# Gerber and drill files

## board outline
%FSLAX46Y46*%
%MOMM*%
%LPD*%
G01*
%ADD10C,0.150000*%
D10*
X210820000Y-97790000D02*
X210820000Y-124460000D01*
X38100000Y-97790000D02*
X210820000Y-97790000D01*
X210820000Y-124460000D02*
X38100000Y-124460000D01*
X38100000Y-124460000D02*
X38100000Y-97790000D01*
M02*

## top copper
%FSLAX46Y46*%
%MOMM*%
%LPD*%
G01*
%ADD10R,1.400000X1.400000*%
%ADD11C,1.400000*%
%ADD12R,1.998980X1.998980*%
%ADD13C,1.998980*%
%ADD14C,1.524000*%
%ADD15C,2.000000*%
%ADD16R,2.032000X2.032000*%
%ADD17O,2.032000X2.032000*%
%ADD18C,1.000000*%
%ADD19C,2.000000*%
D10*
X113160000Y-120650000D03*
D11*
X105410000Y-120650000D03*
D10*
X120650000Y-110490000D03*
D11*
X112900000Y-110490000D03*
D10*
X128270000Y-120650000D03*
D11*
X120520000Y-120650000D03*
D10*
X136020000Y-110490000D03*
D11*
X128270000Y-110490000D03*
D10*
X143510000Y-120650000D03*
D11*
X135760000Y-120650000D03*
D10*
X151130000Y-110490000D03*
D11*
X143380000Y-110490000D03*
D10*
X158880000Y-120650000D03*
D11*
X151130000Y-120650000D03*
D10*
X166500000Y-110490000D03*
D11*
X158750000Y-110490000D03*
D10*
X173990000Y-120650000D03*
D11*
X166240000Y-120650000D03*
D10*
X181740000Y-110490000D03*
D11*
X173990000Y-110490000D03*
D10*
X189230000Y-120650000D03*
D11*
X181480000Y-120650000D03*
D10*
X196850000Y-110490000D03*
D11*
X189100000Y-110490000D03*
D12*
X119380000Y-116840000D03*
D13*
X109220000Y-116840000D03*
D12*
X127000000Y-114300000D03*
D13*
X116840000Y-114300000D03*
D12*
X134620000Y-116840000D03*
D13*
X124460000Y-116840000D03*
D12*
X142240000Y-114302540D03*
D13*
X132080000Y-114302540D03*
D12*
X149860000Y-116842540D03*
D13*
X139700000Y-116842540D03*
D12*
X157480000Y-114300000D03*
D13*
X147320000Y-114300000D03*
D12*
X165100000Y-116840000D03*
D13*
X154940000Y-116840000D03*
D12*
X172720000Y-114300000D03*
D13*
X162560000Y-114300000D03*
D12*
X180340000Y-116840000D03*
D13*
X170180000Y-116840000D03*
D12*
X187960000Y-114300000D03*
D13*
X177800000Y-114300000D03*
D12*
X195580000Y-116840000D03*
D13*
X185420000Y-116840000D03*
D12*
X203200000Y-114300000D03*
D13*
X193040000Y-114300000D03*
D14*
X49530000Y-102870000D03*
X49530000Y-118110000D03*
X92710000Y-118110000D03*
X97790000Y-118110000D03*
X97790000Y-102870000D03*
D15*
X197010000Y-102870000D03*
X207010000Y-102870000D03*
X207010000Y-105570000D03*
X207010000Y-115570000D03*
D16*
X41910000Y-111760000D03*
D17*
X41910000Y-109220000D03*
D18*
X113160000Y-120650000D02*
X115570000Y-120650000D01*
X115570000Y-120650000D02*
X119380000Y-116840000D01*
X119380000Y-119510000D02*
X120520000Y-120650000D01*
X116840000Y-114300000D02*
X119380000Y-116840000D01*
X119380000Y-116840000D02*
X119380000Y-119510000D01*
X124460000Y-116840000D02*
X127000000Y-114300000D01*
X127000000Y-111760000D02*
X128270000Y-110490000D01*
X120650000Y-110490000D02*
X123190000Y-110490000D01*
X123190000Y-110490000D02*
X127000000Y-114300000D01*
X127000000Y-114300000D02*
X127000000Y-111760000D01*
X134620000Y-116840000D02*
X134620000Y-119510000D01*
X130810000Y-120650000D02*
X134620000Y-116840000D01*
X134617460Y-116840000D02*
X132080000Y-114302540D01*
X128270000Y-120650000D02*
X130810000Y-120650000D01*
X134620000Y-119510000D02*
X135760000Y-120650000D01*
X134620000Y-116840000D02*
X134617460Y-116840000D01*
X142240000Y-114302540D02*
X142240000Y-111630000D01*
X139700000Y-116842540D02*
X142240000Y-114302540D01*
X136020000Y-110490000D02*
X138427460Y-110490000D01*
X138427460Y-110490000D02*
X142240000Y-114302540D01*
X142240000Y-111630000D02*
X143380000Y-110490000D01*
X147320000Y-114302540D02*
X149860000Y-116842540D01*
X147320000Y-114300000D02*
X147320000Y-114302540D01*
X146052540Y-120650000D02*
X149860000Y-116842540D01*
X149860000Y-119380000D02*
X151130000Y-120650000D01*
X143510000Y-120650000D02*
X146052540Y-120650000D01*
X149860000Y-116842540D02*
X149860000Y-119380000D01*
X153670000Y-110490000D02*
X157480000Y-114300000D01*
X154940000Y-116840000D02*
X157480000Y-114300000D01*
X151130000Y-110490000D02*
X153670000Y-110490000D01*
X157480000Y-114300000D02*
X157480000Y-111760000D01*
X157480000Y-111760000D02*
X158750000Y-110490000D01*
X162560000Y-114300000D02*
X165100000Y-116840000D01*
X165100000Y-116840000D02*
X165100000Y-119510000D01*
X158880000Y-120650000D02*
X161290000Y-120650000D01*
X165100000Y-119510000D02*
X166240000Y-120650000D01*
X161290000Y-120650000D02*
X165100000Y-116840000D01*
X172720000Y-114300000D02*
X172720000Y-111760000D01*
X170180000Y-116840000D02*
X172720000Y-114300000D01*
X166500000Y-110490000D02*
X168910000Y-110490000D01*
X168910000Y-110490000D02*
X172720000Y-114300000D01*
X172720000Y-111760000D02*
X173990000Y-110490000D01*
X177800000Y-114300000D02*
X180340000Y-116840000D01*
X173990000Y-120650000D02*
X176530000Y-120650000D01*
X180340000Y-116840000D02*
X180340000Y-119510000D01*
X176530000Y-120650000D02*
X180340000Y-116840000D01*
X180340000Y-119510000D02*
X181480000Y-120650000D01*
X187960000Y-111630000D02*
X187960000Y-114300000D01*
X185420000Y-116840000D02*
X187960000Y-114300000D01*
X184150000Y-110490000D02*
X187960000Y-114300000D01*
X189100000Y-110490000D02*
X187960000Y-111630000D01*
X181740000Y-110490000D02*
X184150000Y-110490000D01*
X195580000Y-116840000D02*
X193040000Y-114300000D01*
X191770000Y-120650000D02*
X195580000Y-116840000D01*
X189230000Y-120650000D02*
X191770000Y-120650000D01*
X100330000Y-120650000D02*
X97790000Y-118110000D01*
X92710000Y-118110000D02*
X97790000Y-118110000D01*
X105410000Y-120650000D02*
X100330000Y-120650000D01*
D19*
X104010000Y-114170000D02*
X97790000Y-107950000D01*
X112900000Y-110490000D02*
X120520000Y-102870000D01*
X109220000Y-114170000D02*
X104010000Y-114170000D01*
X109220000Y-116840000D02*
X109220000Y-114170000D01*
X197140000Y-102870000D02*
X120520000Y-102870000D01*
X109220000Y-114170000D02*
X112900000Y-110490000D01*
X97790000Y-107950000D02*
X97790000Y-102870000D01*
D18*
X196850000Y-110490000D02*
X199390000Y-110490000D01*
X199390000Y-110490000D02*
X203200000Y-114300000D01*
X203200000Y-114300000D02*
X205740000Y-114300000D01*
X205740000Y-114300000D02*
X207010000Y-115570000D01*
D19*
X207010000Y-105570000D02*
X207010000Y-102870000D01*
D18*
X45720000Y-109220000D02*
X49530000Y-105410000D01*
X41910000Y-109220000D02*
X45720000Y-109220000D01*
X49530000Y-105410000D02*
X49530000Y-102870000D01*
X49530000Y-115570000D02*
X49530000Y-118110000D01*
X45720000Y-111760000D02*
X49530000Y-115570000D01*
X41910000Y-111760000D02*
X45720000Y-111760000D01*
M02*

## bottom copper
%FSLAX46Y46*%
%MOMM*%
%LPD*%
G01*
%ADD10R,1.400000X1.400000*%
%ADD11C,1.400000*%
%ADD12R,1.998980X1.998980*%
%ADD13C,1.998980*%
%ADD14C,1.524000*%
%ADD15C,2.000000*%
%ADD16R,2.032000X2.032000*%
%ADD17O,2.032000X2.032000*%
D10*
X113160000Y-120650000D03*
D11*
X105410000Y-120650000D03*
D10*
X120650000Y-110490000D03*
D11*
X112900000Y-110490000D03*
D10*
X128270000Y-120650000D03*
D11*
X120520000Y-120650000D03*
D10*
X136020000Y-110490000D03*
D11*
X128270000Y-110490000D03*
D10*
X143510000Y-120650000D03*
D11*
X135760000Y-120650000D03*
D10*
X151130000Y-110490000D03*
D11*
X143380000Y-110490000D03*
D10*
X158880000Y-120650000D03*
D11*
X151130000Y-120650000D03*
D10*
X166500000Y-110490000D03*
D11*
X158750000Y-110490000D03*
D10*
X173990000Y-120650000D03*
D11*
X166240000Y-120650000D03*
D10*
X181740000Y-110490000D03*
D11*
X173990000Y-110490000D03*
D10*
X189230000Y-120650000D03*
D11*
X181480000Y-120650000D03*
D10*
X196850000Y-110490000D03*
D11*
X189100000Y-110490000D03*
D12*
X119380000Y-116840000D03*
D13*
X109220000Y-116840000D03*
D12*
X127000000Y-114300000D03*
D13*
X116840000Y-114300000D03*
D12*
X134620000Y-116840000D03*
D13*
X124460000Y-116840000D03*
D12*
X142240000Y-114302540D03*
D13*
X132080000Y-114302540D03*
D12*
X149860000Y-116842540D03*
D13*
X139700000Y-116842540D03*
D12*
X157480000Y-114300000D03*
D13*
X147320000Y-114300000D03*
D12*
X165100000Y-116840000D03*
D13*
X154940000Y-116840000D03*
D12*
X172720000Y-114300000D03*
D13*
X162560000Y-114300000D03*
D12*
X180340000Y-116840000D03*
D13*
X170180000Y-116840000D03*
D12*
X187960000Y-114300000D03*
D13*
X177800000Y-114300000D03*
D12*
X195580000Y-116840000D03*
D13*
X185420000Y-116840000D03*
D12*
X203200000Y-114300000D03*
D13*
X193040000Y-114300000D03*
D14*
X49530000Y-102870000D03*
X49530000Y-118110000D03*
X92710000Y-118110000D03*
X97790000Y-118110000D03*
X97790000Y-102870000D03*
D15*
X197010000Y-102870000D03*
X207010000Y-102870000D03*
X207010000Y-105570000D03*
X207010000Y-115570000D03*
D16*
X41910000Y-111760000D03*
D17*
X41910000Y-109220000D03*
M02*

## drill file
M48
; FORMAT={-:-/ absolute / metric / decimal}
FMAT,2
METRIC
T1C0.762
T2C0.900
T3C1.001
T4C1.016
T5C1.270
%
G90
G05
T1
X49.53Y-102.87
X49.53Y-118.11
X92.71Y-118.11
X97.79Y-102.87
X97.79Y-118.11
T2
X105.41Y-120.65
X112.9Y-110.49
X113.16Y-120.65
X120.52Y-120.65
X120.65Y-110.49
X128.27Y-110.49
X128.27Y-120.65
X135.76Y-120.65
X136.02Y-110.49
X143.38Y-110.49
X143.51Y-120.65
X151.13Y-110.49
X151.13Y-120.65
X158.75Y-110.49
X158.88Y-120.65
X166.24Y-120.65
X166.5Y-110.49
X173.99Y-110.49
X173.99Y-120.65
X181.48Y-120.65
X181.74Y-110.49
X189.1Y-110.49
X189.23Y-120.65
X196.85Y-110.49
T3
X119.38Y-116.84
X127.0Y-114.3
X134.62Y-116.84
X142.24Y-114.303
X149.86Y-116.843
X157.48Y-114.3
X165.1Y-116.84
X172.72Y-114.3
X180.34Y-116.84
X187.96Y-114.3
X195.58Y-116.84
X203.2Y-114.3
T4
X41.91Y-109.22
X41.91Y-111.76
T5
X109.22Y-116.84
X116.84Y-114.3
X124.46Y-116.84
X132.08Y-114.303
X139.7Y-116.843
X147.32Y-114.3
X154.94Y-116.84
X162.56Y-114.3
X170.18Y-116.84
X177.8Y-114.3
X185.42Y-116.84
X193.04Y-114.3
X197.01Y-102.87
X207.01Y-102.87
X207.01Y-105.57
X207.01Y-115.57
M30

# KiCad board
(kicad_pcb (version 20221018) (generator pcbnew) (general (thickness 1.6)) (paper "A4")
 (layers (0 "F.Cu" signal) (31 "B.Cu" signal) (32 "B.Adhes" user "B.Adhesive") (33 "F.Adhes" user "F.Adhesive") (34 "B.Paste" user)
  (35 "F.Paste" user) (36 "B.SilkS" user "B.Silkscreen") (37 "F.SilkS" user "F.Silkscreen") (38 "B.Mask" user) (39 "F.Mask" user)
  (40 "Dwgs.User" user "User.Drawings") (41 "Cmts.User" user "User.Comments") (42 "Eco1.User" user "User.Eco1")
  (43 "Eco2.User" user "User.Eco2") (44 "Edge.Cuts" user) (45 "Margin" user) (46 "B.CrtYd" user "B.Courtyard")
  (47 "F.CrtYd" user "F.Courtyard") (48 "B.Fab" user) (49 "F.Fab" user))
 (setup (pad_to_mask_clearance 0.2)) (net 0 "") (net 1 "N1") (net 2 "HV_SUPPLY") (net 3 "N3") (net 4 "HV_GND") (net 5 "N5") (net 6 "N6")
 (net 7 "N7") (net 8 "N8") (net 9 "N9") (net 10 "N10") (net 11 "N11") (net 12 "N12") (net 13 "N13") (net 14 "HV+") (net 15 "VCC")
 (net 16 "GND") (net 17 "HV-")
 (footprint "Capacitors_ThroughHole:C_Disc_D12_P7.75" (layer "F.Cu") (at 113.16 120.65 180)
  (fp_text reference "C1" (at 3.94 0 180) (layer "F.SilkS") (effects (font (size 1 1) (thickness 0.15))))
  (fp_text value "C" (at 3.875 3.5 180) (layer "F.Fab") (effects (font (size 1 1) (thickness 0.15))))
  (pad "1" thru_hole rect (at 0 0 180) (size 1.4 1.4) (drill 0.9) (layers "*.Cu" "*.Mask" "F.SilkS") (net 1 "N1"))
  (pad "2" thru_hole circle (at 7.75 0 180) (size 1.4 1.4) (drill 0.9) (layers "*.Cu" "*.Mask" "F.SilkS") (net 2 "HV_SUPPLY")))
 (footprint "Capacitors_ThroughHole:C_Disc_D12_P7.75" (layer "F.Cu") (at 120.65 110.49 180)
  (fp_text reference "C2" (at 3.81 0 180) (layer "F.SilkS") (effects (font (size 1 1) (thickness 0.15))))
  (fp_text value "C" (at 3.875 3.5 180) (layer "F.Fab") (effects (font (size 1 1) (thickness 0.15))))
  (pad "1" thru_hole rect (at 0 0 180) (size 1.4 1.4) (drill 0.9) (layers "*.Cu" "*.Mask" "F.SilkS") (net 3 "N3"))
  (pad "2" thru_hole circle (at 7.75 0 180) (size 1.4 1.4) (drill 0.9) (layers "*.Cu" "*.Mask" "F.SilkS") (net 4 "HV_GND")))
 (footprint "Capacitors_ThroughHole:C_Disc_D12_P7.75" (layer "F.Cu") (at 128.27 120.65 180)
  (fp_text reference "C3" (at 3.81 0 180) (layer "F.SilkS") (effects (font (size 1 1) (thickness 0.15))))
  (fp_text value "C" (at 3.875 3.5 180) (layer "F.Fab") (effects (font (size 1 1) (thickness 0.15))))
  (pad "1" thru_hole rect (at 0 0 180) (size 1.4 1.4) (drill 0.9) (layers "*.Cu" "*.Mask" "F.SilkS") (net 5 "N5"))
  (pad "2" thru_hole circle (at 7.75 0 180) (size 1.4 1.4) (drill 0.9) (layers "*.Cu" "*.Mask" "F.SilkS") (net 1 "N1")))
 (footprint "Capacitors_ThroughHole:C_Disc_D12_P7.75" (layer "F.Cu") (at 136.02 110.49 180)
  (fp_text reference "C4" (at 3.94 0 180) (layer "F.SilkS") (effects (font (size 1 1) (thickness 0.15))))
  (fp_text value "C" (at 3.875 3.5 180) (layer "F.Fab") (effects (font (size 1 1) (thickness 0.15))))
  (pad "1" thru_hole rect (at 0 0 180) (size 1.4 1.4) (drill 0.9) (layers "*.Cu" "*.Mask" "F.SilkS") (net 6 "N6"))
  (pad "2" thru_hole circle (at 7.75 0 180) (size 1.4 1.4) (drill 0.9) (layers "*.Cu" "*.Mask" "F.SilkS") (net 3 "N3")))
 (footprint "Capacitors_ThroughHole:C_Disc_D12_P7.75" (layer "F.Cu") (at 143.51 120.65 180)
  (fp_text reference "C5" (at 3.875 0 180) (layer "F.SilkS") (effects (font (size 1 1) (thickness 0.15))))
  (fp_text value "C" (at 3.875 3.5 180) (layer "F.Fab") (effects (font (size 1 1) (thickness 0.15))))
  (pad "1" thru_hole rect (at 0 0 180) (size 1.4 1.4) (drill 0.9) (layers "*.Cu" "*.Mask" "F.SilkS") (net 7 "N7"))
  (pad "2" thru_hole circle (at 7.75 0 180) (size 1.4 1.4) (drill 0.9) (layers "*.Cu" "*.Mask" "F.SilkS") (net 5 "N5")))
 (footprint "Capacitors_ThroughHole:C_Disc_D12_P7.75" (layer "F.Cu") (at 151.13 110.49 180)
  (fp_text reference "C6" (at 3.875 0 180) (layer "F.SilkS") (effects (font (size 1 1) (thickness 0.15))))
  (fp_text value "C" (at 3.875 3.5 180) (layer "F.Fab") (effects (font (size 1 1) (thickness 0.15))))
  (pad "1" thru_hole rect (at 0 0 180) (size 1.4 1.4) (drill 0.9) (layers "*.Cu" "*.Mask" "F.SilkS") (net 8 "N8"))
  (pad "2" thru_hole circle (at 7.75 0 180) (size 1.4 1.4) (drill 0.9) (layers "*.Cu" "*.Mask" "F.SilkS") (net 6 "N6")))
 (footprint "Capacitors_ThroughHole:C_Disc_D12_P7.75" (layer "F.Cu") (at 158.88 120.65 180)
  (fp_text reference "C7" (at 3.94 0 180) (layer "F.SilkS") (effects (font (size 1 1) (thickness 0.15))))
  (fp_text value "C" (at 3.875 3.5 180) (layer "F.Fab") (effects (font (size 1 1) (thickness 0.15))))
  (pad "1" thru_hole rect (at 0 0 180) (size 1.4 1.4) (drill 0.9) (layers "*.Cu" "*.Mask" "F.SilkS") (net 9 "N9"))
  (pad "2" thru_hole circle (at 7.75 0 180) (size 1.4 1.4) (drill 0.9) (layers "*.Cu" "*.Mask" "F.SilkS") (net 7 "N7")))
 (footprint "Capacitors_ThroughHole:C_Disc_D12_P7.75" (layer "F.Cu") (at 166.5 110.49 180)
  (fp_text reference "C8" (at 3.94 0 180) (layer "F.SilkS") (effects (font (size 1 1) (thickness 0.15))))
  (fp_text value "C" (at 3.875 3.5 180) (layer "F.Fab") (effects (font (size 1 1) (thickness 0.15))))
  (pad "1" thru_hole rect (at 0 0 180) (size 1.4 1.4) (drill 0.9) (layers "*.Cu" "*.Mask" "F.SilkS") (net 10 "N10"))
  (pad "2" thru_hole circle (at 7.75 0 180) (size 1.4 1.4) (drill 0.9) (layers "*.Cu" "*.Mask" "F.SilkS") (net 8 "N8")))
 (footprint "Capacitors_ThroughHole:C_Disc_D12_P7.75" (layer "F.Cu") (at 173.99 120.65 180)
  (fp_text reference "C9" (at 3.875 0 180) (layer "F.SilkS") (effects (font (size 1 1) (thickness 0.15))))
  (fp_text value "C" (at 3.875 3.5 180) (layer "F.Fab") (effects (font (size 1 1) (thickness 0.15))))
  (pad "1" thru_hole rect (at 0 0 180) (size 1.4 1.4) (drill 0.9) (layers "*.Cu" "*.Mask" "F.SilkS") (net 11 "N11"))
  (pad "2" thru_hole circle (at 7.75 0 180) (size 1.4 1.4) (drill 0.9) (layers "*.Cu" "*.Mask" "F.SilkS") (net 9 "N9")))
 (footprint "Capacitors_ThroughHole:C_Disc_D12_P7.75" (layer "F.Cu") (at 181.74 110.49 180)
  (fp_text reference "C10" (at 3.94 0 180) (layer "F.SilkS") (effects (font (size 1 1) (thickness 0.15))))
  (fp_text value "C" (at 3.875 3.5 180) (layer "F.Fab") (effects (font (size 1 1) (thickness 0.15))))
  (pad "1" thru_hole rect (at 0 0 180) (size 1.4 1.4) (drill 0.9) (layers "*.Cu" "*.Mask" "F.SilkS") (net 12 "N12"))
  (pad "2" thru_hole circle (at 7.75 0 180) (size 1.4 1.4) (drill 0.9) (layers "*.Cu" "*.Mask" "F.SilkS") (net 10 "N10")))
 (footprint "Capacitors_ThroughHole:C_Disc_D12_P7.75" (layer "F.Cu") (at 189.23 120.65 180)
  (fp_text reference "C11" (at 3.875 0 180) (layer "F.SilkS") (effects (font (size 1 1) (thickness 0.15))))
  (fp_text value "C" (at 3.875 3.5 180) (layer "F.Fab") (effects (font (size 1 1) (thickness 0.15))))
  (pad "1" thru_hole rect (at 0 0 180) (size 1.4 1.4) (drill 0.9) (layers "*.Cu" "*.Mask" "F.SilkS") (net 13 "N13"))
  (pad "2" thru_hole circle (at 7.75 0 180) (size 1.4 1.4) (drill 0.9) (layers "*.Cu" "*.Mask" "F.SilkS") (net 11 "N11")))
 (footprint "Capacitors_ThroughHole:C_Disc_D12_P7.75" (layer "F.Cu") (at 196.85 110.49 180)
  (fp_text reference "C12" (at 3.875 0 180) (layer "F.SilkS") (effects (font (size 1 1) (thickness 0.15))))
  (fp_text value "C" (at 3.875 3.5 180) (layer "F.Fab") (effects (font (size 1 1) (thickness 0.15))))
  (pad "1" thru_hole rect (at 0 0 180) (size 1.4 1.4) (drill 0.9) (layers "*.Cu" "*.Mask" "F.SilkS") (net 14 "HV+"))
  (pad "2" thru_hole circle (at 7.75 0 180) (size 1.4 1.4) (drill 0.9) (layers "*.Cu" "*.Mask" "F.SilkS") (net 12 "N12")))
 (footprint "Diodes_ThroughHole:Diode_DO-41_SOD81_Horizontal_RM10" (layer "F.Cu") (at 119.38 116.83746 180)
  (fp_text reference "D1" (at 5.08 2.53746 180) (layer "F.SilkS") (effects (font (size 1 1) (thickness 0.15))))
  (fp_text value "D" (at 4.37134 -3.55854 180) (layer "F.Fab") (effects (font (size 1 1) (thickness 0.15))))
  (pad "1" thru_hole rect (at 0 -0.00254) (size 1.99898 1.99898) (drill 1.00076) (layers "*.Cu" "*.Mask" "F.SilkS") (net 1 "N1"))
  (pad "2" thru_hole circle (at 10.16 -0.00254) (size 1.99898 1.99898) (drill 1.27) (layers "*.Cu" "*.Mask" "F.SilkS") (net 4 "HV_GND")))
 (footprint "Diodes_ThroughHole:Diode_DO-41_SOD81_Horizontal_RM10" (layer "F.Cu") (at 127 114.29746 180)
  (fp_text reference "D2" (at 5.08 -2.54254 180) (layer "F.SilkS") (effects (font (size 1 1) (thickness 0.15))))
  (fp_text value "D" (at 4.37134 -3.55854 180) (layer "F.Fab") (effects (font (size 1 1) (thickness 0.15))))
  (pad "1" thru_hole rect (at 0 -0.00254) (size 1.99898 1.99898) (drill 1.00076) (layers "*.Cu" "*.Mask" "F.SilkS") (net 3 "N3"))
  (pad "2" thru_hole circle (at 10.16 -0.00254) (size 1.99898 1.99898) (drill 1.27) (layers "*.Cu" "*.Mask" "F.SilkS") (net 1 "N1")))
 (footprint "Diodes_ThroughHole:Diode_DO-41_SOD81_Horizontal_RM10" (layer "F.Cu") (at 134.62 116.83746 180)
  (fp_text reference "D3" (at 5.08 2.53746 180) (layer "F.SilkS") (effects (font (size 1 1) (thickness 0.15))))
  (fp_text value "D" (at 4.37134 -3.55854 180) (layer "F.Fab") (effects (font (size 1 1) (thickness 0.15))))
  (pad "1" thru_hole rect (at 0 -0.00254) (size 1.99898 1.99898) (drill 1.00076) (layers "*.Cu" "*.Mask" "F.SilkS") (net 5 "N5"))
  (pad "2" thru_hole circle (at 10.16 -0.00254) (size 1.99898 1.99898) (drill 1.27) (layers "*.Cu" "*.Mask" "F.SilkS") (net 3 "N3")))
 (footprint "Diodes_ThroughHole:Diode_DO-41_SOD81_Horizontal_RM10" (layer "F.Cu") (at 142.24 114.3 180)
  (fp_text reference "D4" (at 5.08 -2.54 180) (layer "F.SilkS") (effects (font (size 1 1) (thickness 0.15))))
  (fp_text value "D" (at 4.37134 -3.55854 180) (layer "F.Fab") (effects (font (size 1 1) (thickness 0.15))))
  (pad "1" thru_hole rect (at 0 -0.00254) (size 1.99898 1.99898) (drill 1.00076) (layers "*.Cu" "*.Mask" "F.SilkS") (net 6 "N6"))
  (pad "2" thru_hole circle (at 10.16 -0.00254) (size 1.99898 1.99898) (drill 1.27) (layers "*.Cu" "*.Mask" "F.SilkS") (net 5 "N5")))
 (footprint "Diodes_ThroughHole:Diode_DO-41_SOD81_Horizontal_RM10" (layer "F.Cu") (at 149.86 116.84 180)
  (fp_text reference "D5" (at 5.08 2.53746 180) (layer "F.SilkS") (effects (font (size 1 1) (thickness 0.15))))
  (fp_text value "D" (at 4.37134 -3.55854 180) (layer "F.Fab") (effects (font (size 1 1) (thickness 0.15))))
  (pad "1" thru_hole rect (at 0 -0.00254) (size 1.99898 1.99898) (drill 1.00076) (layers "*.Cu" "*.Mask" "F.SilkS") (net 7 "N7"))
  (pad "2" thru_hole circle (at 10.16 -0.00254) (size 1.99898 1.99898) (drill 1.27) (layers "*.Cu" "*.Mask" "F.SilkS") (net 6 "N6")))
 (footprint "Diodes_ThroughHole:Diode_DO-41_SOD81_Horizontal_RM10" (layer "F.Cu") (at 157.48 114.29746 180)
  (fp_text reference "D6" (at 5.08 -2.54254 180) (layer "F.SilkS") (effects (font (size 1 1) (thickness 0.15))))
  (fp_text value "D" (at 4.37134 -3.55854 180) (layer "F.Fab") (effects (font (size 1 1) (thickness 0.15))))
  (pad "1" thru_hole rect (at 0 -0.00254) (size 1.99898 1.99898) (drill 1.00076) (layers "*.Cu" "*.Mask" "F.SilkS") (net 8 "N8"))
  (pad "2" thru_hole circle (at 10.16 -0.00254) (size 1.99898 1.99898) (drill 1.27) (layers "*.Cu" "*.Mask" "F.SilkS") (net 7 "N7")))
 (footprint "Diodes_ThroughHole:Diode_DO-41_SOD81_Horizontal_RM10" (layer "F.Cu") (at 165.1 116.83746 180)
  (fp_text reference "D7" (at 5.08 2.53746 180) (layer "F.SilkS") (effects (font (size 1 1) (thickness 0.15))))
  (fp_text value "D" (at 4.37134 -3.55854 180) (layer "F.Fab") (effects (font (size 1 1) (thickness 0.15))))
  (pad "1" thru_hole rect (at 0 -0.00254) (size 1.99898 1.99898) (drill 1.00076) (layers "*.Cu" "*.Mask" "F.SilkS") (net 9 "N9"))
  (pad "2" thru_hole circle (at 10.16 -0.00254) (size 1.99898 1.99898) (drill 1.27) (layers "*.Cu" "*.Mask" "F.SilkS") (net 8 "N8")))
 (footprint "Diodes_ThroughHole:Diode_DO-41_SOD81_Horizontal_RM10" (layer "F.Cu") (at 172.72 114.29746 180)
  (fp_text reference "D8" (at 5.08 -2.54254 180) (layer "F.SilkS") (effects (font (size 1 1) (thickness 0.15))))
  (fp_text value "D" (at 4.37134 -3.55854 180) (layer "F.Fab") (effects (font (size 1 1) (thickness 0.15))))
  (pad "1" thru_hole rect (at 0 -0.00254) (size 1.99898 1.99898) (drill 1.00076) (layers "*.Cu" "*.Mask" "F.SilkS") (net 10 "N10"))
  (pad "2" thru_hole circle (at 10.16 -0.00254) (size 1.99898 1.99898) (drill 1.27) (layers "*.Cu" "*.Mask" "F.SilkS") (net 9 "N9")))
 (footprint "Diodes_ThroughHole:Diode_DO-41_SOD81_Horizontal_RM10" (layer "F.Cu") (at 180.34 116.83746 180)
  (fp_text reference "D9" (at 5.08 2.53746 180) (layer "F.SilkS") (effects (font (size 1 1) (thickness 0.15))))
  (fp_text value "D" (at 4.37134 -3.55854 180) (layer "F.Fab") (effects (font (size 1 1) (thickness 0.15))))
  (pad "1" thru_hole rect (at 0 -0.00254) (size 1.99898 1.99898) (drill 1.00076) (layers "*.Cu" "*.Mask" "F.SilkS") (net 11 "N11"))
  (pad "2" thru_hole circle (at 10.16 -0.00254) (size 1.99898 1.99898) (drill 1.27) (layers "*.Cu" "*.Mask" "F.SilkS") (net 10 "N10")))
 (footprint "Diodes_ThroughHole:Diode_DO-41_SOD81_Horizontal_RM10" (layer "F.Cu") (at 187.96 114.29746 180)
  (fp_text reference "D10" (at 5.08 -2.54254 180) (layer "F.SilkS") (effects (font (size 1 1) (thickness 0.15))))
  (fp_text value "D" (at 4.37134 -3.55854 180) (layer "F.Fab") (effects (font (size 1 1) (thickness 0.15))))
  (pad "1" thru_hole rect (at 0 -0.00254) (size 1.99898 1.99898) (drill 1.00076) (layers "*.Cu" "*.Mask" "F.SilkS") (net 12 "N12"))
  (pad "2" thru_hole circle (at 10.16 -0.00254) (size 1.99898 1.99898) (drill 1.27) (layers "*.Cu" "*.Mask" "F.SilkS") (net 11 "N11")))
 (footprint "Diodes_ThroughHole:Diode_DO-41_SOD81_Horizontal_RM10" (layer "F.Cu") (at 195.58 116.83746 180)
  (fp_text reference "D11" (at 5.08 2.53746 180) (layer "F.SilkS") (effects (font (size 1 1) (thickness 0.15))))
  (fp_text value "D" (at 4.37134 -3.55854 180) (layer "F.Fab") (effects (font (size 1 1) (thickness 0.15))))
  (pad "1" thru_hole rect (at 0 -0.00254) (size 1.99898 1.99898) (drill 1.00076) (layers "*.Cu" "*.Mask" "F.SilkS") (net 13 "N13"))
  (pad "2" thru_hole circle (at 10.16 -0.00254) (size 1.99898 1.99898) (drill 1.27) (layers "*.Cu" "*.Mask" "F.SilkS") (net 12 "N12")))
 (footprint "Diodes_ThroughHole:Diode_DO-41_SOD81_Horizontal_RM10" (layer "F.Cu") (at 203.2 114.29746 180)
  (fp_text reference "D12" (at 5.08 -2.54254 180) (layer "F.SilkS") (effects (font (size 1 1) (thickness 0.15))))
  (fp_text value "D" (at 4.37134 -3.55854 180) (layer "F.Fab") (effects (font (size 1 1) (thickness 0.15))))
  (pad "1" thru_hole rect (at 0 -0.00254) (size 1.99898 1.99898) (drill 1.00076) (layers "*.Cu" "*.Mask" "F.SilkS") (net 14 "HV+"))
  (pad "2" thru_hole circle (at 10.16 -0.00254) (size 1.99898 1.99898) (drill 1.27) (layers "*.Cu" "*.Mask" "F.SilkS") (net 13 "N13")))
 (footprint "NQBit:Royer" (layer "F.Cu") (at 74.93 110.49)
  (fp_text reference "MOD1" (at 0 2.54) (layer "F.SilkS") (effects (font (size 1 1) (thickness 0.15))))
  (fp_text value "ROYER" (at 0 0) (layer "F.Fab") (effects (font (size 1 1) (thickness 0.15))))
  (pad "1" thru_hole circle (at -25.4 -7.62) (size 1.524 1.524) (drill 0.762) (layers "*.Cu" "*.Mask" "F.SilkS") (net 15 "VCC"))
  (pad "2" thru_hole circle (at -25.4 7.62) (size 1.524 1.524) (drill 0.762) (layers "*.Cu" "*.Mask" "F.SilkS") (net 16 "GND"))
  (pad "3" thru_hole circle (at 17.78 7.62) (size 1.524 1.524) (drill 0.762) (layers "*.Cu" "*.Mask" "F.SilkS") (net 2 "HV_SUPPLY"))
  (pad "4" thru_hole circle (at 22.86 7.62) (size 1.524 1.524) (drill 0.762) (layers "*.Cu" "*.Mask" "F.SilkS") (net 2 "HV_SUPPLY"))
  (pad "5" thru_hole circle (at 22.86 -7.62) (size 1.524 1.524) (drill 0.762) (layers "*.Cu" "*.Mask" "F.SilkS") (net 4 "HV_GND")))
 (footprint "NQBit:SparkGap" (layer "F.Cu") (at 197.01 102.87)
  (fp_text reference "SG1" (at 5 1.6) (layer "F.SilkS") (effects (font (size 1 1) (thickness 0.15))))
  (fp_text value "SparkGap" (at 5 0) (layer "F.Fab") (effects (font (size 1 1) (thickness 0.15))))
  (pad "1" thru_hole circle (at 0 0) (size 2 2) (drill 1.27) (layers "*.Cu" "*.Mask" "F.SilkS") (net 4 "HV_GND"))
  (pad "2" thru_hole circle (at 10 0) (size 2 2) (drill 1.27) (layers "*.Cu" "*.Mask" "F.SilkS") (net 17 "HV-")))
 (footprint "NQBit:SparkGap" (layer "F.Cu") (at 207.01 105.57 -90)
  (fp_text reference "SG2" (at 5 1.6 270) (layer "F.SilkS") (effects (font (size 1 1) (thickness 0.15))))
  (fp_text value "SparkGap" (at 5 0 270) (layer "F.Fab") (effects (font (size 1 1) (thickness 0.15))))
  (pad "1" thru_hole circle (at 0 0 270) (size 2 2) (drill 1.27) (layers "*.Cu" "*.Mask" "F.SilkS") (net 17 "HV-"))
  (pad "2" thru_hole circle (at 10 0 270) (size 2 2) (drill 1.27) (layers "*.Cu" "*.Mask" "F.SilkS") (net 14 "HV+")))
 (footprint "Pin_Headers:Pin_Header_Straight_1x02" (layer "F.Cu") (at 41.91 111.76 180)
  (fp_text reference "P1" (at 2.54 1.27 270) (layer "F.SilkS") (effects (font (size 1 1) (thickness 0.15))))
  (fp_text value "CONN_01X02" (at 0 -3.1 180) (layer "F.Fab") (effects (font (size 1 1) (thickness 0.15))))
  (pad "1" thru_hole rect (at 0 0 180) (size 2.032 2.032) (drill 1.016) (layers "*.Cu" "*.Mask" "F.SilkS") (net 16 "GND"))
  (pad "2" thru_hole oval (at 0 2.54 180) (size 2.032 2.032) (drill 1.016) (layers "*.Cu" "*.Mask" "F.SilkS") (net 15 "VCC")))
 (gr_line (start 210.82 97.79) (end 210.82 124.46) (stroke (width 0.15) (type solid)) (layer "Edge.Cuts"))
 (gr_line (start 38.1 97.79) (end 210.82 97.79) (stroke (width 0.15) (type solid)) (layer "Edge.Cuts"))
 (gr_line (start 210.82 124.46) (end 38.1 124.46) (stroke (width 0.15) (type solid)) (layer "Edge.Cuts"))
 (gr_line (start 38.1 124.46) (end 38.1 97.79) (stroke (width 0.15) (type solid)) (layer "Edge.Cuts"))
 (segment (start 113.16 120.65) (end 115.57 120.65) (width 1) (layer "F.Cu") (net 1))
 (segment (start 115.57 120.65) (end 119.38 116.84) (width 1) (layer "F.Cu") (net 1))
 (segment (start 119.38 119.51) (end 120.52 120.65) (width 1) (layer "F.Cu") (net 1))
 (segment (start 116.84 114.3) (end 119.38 116.84) (width 1) (layer "F.Cu") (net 1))
 (segment (start 119.38 116.84) (end 119.38 119.51) (width 1) (layer "F.Cu") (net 1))
 (segment (start 124.46 116.84) (end 127 114.3) (width 1) (layer "F.Cu") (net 3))
 (segment (start 127 111.76) (end 128.27 110.49) (width 1) (layer "F.Cu") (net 3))
 (segment (start 120.65 110.49) (end 123.19 110.49) (width 1) (layer "F.Cu") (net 3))
 (segment (start 123.19 110.49) (end 127 114.3) (width 1) (layer "F.Cu") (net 3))
 (segment (start 127 114.3) (end 127 111.76) (width 1) (layer "F.Cu") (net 3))
 (segment (start 134.62 116.84) (end 134.62 119.51) (width 1) (layer "F.Cu") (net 5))
 (segment (start 130.81 120.65) (end 134.62 116.84) (width 1) (layer "F.Cu") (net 5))
 (segment (start 134.61746 116.84) (end 132.08 114.30254) (width 1) (layer "F.Cu") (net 5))
 (segment (start 128.27 120.65) (end 130.81 120.65) (width 1) (layer "F.Cu") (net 5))
 (segment (start 134.62 119.51) (end 135.76 120.65) (width 1) (layer "F.Cu") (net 5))
 (segment (start 134.62 116.84) (end 134.61746 116.84) (width 1) (layer "F.Cu") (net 5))
 (segment (start 142.24 114.30254) (end 142.24 111.63) (width 1) (layer "F.Cu") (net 6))
 (segment (start 139.7 116.84254) (end 142.24 114.30254) (width 1) (layer "F.Cu") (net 6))
 (segment (start 136.02 110.49) (end 138.42746 110.49) (width 1) (layer "F.Cu") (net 6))
 (segment (start 138.42746 110.49) (end 142.24 114.30254) (width 1) (layer "F.Cu") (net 6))
 (segment (start 142.24 111.63) (end 143.38 110.49) (width 1) (layer "F.Cu") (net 6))
 (segment (start 147.32 114.30254) (end 149.86 116.84254) (width 1) (layer "F.Cu") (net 7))
 (segment (start 147.32 114.3) (end 147.32 114.30254) (width 1) (layer "F.Cu") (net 7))
 (segment (start 146.05254 120.65) (end 149.86 116.84254) (width 1) (layer "F.Cu") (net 7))
 (segment (start 149.86 119.38) (end 151.13 120.65) (width 1) (layer "F.Cu") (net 7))
 (segment (start 143.51 120.65) (end 146.05254 120.65) (width 1) (layer "F.Cu") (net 7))
 (segment (start 149.86 116.84254) (end 149.86 119.38) (width 1) (layer "F.Cu") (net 7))
 (segment (start 153.67 110.49) (end 157.48 114.3) (width 1) (layer "F.Cu") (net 8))
 (segment (start 154.94 116.84) (end 157.48 114.3) (width 1) (layer "F.Cu") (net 8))
 (segment (start 151.13 110.49) (end 153.67 110.49) (width 1) (layer "F.Cu") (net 8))
 (segment (start 157.48 114.3) (end 157.48 111.76) (width 1) (layer "F.Cu") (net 8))
 (segment (start 157.48 111.76) (end 158.75 110.49) (width 1) (layer "F.Cu") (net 8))
 (segment (start 162.56 114.3) (end 165.1 116.84) (width 1) (layer "F.Cu") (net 9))
 (segment (start 165.1 116.84) (end 165.1 119.51) (width 1) (layer "F.Cu") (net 9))
 (segment (start 158.88 120.65) (end 161.29 120.65) (width 1) (layer "F.Cu") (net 9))
 (segment (start 165.1 119.51) (end 166.24 120.65) (width 1) (layer "F.Cu") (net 9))
 (segment (start 161.29 120.65) (end 165.1 116.84) (width 1) (layer "F.Cu") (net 9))
 (segment (start 172.72 114.3) (end 172.72 111.76) (width 1) (layer "F.Cu") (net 10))
 (segment (start 170.18 116.84) (end 172.72 114.3) (width 1) (layer "F.Cu") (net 10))
 (segment (start 166.5 110.49) (end 168.91 110.49) (width 1) (layer "F.Cu") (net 10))
 (segment (start 168.91 110.49) (end 172.72 114.3) (width 1) (layer "F.Cu") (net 10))
 (segment (start 172.72 111.76) (end 173.99 110.49) (width 1) (layer "F.Cu") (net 10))
 (segment (start 177.8 114.3) (end 180.34 116.84) (width 1) (layer "F.Cu") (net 11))
 (segment (start 173.99 120.65) (end 176.53 120.65) (width 1) (layer "F.Cu") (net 11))
 (segment (start 180.34 116.84) (end 180.34 119.51) (width 1) (layer "F.Cu") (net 11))
 (segment (start 176.53 120.65) (end 180.34 116.84) (width 1) (layer "F.Cu") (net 11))
 (segment (start 180.34 119.51) (end 181.48 120.65) (width 1) (layer "F.Cu") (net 11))
 (segment (start 187.96 111.63) (end 187.96 114.3) (width 1) (layer "F.Cu") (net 12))
 (segment (start 185.42 116.84) (end 187.96 114.3) (width 1) (layer "F.Cu") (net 12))
 (segment (start 184.15 110.49) (end 187.96 114.3) (width 1) (layer "F.Cu") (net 12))
 (segment (start 189.1 110.49) (end 187.96 111.63) (width 1) (layer "F.Cu") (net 12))
 (segment (start 181.74 110.49) (end 184.15 110.49) (width 1) (layer "F.Cu") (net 12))
 (segment (start 195.58 116.84) (end 193.04 114.3) (width 1) (layer "F.Cu") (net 13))
 (segment (start 191.77 120.65) (end 195.58 116.84) (width 1) (layer "F.Cu") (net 13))
 (segment (start 189.23 120.65) (end 191.77 120.65) (width 1) (layer "F.Cu") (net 13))
 (segment (start 100.33 120.65) (end 97.79 118.11) (width 1) (layer "F.Cu") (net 2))
 (segment (start 92.71 118.11) (end 97.79 118.11) (width 1) (layer "F.Cu") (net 2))
 (segment (start 105.41 120.65) (end 100.33 120.65) (width 1) (layer "F.Cu") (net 2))
 (segment (start 104.01 114.17) (end 97.79 107.95) (width 2) (layer "F.Cu") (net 4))
 (segment (start 112.9 110.49) (end 120.52 102.87) (width 2) (layer "F.Cu") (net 4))
 (segment (start 109.22 114.17) (end 104.01 114.17) (width 2) (layer "F.Cu") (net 4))
 (segment (start 109.22 116.84) (end 109.22 114.17) (width 2) (layer "F.Cu") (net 4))
 (segment (start 197.14 102.87) (end 120.52 102.87) (width 2) (layer "F.Cu") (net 4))
 (segment (start 109.22 114.17) (end 112.9 110.49) (width 2) (layer "F.Cu") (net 4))
 (segment (start 97.79 107.95) (end 97.79 102.87) (width 2) (layer "F.Cu") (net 4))
 (segment (start 196.85 110.49) (end 199.39 110.49) (width 1) (layer "F.Cu") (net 14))
 (segment (start 199.39 110.49) (end 203.2 114.3) (width 1) (layer "F.Cu") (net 14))
 (segment (start 203.2 114.3) (end 205.74 114.3) (width 1) (layer "F.Cu") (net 14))
 (segment (start 205.74 114.3) (end 207.01 115.57) (width 1) (layer "F.Cu") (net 14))
 (segment (start 207.01 105.57) (end 207.01 102.87) (width 2) (layer "F.Cu") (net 17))
 (segment (start 45.72 109.22) (end 49.53 105.41) (width 1) (layer "F.Cu") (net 15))
 (segment (start 41.91 109.22) (end 45.72 109.22) (width 1) (layer "F.Cu") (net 15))
 (segment (start 49.53 105.41) (end 49.53 102.87) (width 1) (layer "F.Cu") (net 15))
 (segment (start 49.53 115.57) (end 49.53 118.11) (width 1) (layer "F.Cu") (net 16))
 (segment (start 45.72 111.76) (end 49.53 115.57) (width 1) (layer "F.Cu") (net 16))
 (segment (start 41.91 111.76) (end 45.72 111.76) (width 1) (layer "F.Cu") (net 16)))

